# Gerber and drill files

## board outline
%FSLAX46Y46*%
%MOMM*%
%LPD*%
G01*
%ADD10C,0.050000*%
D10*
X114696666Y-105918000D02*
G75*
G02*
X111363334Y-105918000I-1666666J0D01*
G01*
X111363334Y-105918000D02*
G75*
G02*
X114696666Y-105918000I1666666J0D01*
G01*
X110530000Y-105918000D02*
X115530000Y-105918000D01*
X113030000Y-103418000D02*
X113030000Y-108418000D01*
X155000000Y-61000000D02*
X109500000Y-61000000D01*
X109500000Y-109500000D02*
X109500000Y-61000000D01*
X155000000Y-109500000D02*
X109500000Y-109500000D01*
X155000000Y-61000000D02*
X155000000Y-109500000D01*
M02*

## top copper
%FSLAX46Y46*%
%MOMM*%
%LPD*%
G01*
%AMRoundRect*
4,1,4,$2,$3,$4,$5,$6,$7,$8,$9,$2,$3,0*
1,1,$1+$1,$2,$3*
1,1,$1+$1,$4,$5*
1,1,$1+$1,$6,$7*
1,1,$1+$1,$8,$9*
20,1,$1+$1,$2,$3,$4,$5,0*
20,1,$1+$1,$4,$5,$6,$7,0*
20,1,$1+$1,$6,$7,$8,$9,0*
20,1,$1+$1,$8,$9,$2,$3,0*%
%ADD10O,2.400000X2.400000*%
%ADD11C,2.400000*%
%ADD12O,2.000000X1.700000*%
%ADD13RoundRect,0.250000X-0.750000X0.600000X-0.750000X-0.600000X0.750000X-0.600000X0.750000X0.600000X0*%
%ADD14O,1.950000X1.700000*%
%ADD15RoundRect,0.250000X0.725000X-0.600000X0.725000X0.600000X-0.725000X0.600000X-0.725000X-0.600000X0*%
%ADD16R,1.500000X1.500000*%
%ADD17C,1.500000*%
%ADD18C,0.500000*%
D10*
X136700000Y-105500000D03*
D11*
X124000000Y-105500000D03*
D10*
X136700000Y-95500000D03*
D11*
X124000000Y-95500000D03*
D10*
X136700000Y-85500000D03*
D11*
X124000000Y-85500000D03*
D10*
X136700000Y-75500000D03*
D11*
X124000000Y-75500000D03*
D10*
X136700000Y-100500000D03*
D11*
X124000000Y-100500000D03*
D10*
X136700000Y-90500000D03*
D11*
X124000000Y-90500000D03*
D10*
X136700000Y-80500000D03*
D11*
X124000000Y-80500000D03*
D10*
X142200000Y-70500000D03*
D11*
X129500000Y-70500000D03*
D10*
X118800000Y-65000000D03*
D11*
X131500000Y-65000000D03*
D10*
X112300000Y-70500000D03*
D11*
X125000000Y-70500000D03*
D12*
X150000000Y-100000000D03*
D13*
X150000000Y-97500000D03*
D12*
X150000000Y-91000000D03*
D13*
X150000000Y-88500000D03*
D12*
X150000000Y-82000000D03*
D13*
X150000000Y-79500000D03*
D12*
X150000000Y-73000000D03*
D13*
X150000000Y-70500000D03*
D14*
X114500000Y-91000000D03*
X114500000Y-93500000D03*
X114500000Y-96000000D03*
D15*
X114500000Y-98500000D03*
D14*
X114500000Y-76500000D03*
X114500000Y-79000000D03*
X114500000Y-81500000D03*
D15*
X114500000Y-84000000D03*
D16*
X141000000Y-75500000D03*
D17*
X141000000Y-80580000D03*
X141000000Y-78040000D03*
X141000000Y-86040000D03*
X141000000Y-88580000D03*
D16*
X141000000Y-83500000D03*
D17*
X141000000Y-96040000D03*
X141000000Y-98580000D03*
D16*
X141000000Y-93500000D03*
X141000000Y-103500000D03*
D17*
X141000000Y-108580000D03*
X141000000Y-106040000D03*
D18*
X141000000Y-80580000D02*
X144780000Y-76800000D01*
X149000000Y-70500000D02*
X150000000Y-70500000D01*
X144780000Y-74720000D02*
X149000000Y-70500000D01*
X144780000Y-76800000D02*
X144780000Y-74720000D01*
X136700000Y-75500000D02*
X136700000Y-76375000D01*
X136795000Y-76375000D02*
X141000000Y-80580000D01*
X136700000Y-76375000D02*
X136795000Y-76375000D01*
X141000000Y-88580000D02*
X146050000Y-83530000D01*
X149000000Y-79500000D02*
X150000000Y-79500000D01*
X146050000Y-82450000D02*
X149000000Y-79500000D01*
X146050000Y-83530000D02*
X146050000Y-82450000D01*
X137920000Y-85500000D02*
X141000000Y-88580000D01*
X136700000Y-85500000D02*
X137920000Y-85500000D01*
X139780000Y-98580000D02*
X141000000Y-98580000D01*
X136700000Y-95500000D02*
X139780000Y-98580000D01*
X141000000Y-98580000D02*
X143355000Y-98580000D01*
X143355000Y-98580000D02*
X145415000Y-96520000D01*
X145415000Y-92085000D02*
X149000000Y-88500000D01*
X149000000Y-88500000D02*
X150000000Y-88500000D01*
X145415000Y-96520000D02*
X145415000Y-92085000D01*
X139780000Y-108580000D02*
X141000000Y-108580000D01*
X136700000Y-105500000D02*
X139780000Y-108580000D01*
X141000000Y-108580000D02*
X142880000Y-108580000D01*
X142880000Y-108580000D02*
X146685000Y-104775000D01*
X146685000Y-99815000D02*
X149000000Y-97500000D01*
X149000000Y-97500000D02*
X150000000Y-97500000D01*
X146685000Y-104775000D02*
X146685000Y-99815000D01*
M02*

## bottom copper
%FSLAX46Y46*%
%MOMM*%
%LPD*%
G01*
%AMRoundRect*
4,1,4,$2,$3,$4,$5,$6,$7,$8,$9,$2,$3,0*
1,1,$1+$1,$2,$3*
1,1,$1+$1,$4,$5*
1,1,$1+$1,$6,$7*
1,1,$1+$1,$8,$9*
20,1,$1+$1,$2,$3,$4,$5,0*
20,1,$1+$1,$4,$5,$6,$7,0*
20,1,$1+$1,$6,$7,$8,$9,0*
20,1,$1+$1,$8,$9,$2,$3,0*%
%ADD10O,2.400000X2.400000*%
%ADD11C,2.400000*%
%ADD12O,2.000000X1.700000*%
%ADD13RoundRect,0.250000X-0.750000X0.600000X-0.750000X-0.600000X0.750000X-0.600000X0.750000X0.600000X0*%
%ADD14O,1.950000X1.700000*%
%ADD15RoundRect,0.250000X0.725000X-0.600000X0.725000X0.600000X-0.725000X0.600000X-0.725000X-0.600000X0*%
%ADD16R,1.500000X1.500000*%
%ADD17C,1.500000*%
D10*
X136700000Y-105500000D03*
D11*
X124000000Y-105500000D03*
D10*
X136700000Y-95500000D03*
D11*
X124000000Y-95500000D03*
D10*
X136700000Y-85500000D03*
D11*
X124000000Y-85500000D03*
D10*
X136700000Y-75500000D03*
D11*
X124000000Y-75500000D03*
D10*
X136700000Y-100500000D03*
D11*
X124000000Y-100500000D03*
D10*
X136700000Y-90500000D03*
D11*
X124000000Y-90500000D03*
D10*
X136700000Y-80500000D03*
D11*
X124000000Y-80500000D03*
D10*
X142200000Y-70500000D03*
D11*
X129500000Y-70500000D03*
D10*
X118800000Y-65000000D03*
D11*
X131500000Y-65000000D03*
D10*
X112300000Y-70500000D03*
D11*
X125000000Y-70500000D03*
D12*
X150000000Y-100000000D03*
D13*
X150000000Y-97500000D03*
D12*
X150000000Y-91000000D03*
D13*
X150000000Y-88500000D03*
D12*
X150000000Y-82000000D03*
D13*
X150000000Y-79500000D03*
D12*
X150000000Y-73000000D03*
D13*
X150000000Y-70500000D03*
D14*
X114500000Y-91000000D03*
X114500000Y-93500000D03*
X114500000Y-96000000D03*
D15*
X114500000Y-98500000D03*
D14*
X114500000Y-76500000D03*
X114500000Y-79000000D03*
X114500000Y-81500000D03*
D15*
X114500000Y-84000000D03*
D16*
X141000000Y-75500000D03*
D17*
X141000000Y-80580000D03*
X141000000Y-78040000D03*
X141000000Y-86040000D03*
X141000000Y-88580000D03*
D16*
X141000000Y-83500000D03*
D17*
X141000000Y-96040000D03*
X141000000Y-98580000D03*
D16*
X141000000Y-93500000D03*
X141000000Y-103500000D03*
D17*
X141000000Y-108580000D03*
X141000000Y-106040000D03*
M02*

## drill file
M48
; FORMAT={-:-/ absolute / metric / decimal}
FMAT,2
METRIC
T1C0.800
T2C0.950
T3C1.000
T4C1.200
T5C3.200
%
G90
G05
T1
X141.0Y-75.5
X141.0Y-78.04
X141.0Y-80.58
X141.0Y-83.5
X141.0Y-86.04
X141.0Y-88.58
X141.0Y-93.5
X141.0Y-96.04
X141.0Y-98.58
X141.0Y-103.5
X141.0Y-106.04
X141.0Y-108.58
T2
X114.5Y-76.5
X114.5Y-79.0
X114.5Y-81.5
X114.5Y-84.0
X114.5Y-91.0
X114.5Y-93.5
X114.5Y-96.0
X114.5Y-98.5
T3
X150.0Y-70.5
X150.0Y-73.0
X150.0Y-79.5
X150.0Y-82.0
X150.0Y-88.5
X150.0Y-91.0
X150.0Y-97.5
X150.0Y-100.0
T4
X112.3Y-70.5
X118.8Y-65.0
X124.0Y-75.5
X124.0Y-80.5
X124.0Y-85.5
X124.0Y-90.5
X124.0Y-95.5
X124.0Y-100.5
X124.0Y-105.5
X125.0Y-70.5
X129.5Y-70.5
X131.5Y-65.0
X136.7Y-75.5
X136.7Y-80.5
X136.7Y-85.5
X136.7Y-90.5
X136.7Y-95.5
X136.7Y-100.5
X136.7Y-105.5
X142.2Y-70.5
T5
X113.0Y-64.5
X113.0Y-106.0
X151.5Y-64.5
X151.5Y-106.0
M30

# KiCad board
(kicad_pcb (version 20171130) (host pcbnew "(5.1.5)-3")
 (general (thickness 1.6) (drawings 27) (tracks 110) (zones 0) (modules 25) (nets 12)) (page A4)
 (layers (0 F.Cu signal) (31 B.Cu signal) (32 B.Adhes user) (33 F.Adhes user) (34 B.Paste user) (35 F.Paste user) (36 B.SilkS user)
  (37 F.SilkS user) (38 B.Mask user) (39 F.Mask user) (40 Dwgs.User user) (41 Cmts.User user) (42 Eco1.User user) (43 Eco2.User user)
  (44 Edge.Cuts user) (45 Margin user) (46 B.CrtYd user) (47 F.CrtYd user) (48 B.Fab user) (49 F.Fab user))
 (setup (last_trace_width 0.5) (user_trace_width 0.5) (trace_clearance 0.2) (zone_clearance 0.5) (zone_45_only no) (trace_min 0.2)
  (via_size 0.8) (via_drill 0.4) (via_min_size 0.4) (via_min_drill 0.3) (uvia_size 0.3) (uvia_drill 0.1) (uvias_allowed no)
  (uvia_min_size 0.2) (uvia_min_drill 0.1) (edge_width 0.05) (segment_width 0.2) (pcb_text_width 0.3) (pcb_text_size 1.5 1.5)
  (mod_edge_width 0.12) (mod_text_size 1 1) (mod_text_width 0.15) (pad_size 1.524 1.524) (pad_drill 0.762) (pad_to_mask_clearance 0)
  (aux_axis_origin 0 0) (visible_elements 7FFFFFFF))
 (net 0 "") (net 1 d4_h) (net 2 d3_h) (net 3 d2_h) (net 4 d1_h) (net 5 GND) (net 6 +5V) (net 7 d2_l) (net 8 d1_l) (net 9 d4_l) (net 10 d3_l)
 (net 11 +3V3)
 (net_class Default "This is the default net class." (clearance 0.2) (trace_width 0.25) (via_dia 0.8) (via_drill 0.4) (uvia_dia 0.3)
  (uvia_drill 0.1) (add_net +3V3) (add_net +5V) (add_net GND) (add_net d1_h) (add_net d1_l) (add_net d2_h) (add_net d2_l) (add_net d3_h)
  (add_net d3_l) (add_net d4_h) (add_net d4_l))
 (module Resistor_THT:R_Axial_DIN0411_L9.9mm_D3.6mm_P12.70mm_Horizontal (layer F.Cu) (at 124 105.5)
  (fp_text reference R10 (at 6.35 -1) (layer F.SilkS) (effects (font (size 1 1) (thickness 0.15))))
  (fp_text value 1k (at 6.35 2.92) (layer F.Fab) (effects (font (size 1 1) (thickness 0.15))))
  (pad 2 thru_hole oval (at 12.7 0) (size 2.4 2.4) (drill 1.2) (layers *.Cu *.Mask) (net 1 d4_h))
  (pad 1 thru_hole circle (at 0 0) (size 2.4 2.4) (drill 1.2) (layers *.Cu *.Mask)))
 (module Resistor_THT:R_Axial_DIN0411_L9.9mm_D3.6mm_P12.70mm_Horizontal (layer F.Cu) (at 124 95.5)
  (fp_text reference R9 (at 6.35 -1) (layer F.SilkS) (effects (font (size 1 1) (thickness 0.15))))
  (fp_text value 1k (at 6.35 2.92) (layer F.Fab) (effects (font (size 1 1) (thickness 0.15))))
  (pad 2 thru_hole oval (at 12.7 0) (size 2.4 2.4) (drill 1.2) (layers *.Cu *.Mask) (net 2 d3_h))
  (pad 1 thru_hole circle (at 0 0) (size 2.4 2.4) (drill 1.2) (layers *.Cu *.Mask)))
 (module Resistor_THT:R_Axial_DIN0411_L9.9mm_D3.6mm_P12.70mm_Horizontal (layer F.Cu) (at 124 85.5)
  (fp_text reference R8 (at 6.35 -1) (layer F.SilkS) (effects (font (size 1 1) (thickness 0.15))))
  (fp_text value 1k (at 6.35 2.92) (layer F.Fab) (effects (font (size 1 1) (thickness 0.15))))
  (pad 2 thru_hole oval (at 12.7 0) (size 2.4 2.4) (drill 1.2) (layers *.Cu *.Mask) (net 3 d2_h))
  (pad 1 thru_hole circle (at 0 0) (size 2.4 2.4) (drill 1.2) (layers *.Cu *.Mask)))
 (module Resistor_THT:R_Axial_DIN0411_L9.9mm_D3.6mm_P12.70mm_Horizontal (layer F.Cu) (at 124 75.5)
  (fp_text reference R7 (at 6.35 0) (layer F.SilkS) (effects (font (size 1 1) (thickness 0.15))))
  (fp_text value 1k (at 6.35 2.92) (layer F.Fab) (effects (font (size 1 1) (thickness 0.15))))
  (pad 2 thru_hole oval (at 12.7 0) (size 2.4 2.4) (drill 1.2) (layers *.Cu *.Mask) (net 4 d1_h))
  (pad 1 thru_hole circle (at 0 0) (size 2.4 2.4) (drill 1.2) (layers *.Cu *.Mask)))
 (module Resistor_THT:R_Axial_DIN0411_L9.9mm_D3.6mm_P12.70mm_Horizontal (layer F.Cu) (at 124 100.5)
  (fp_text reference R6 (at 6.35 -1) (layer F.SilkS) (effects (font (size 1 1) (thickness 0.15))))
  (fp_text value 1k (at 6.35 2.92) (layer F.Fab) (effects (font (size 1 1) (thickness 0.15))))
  (pad 2 thru_hole oval (at 12.7 0) (size 2.4 2.4) (drill 1.2) (layers *.Cu *.Mask))
  (pad 1 thru_hole circle (at 0 0) (size 2.4 2.4) (drill 1.2) (layers *.Cu *.Mask)))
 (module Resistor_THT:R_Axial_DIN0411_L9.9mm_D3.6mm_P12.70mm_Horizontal (layer F.Cu) (at 124 90.5)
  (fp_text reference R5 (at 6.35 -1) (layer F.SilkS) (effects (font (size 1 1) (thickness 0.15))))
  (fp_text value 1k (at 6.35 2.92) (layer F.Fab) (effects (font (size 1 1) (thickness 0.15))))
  (pad 2 thru_hole oval (at 12.7 0) (size 2.4 2.4) (drill 1.2) (layers *.Cu *.Mask))
  (pad 1 thru_hole circle (at 0 0) (size 2.4 2.4) (drill 1.2) (layers *.Cu *.Mask)))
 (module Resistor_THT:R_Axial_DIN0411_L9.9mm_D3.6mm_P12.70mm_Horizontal (layer F.Cu) (at 124 80.5)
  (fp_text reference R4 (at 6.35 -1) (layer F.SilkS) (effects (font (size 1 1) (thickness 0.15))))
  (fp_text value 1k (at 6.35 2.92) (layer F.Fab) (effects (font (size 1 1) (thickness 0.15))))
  (pad 2 thru_hole oval (at 12.7 0) (size 2.4 2.4) (drill 1.2) (layers *.Cu *.Mask))
  (pad 1 thru_hole circle (at 0 0) (size 2.4 2.4) (drill 1.2) (layers *.Cu *.Mask)))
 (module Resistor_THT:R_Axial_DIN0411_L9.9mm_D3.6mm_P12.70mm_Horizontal (layer F.Cu) (at 129.5 70.5)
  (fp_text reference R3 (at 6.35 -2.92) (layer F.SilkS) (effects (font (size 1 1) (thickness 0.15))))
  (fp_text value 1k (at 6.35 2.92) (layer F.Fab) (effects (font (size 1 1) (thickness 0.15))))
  (pad 2 thru_hole oval (at 12.7 0) (size 2.4 2.4) (drill 1.2) (layers *.Cu *.Mask))
  (pad 1 thru_hole circle (at 0 0) (size 2.4 2.4) (drill 1.2) (layers *.Cu *.Mask)))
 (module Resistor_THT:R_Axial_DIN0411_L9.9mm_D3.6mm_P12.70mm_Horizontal (layer F.Cu) (at 131.5 65 180)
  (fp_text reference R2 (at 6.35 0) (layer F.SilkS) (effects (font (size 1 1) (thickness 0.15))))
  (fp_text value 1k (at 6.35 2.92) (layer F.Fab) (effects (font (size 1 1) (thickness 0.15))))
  (pad 2 thru_hole oval (at 12.7 0 180) (size 2.4 2.4) (drill 1.2) (layers *.Cu *.Mask))
  (pad 1 thru_hole circle (at 0 0 180) (size 2.4 2.4) (drill 1.2) (layers *.Cu *.Mask)))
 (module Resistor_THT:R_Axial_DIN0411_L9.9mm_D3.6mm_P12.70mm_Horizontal (layer F.Cu) (at 125 70.5 180)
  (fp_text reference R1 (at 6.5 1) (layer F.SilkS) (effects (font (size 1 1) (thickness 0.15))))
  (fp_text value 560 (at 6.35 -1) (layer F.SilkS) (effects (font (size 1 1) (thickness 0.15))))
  (pad 2 thru_hole oval (at 12.7 0 180) (size 2.4 2.4) (drill 1.2) (layers *.Cu *.Mask))
  (pad 1 thru_hole circle (at 0 0 180) (size 2.4 2.4) (drill 1.2) (layers *.Cu *.Mask)))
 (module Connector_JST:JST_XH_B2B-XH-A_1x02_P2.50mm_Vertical (layer F.Cu) (at 150 97.5 270)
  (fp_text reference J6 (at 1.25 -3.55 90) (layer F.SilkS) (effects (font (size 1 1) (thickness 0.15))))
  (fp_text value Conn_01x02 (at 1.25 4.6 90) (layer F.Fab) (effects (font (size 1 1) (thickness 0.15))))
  (pad 2 thru_hole oval (at 2.5 0 270) (size 1.7 2) (drill 1) (layers *.Cu *.Mask))
  (pad 1 thru_hole roundrect (at 0 0 270) (size 1.7 2) (drill 1) (layers *.Cu *.Mask) (roundrect_rratio 0.1470588235294118) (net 1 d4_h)))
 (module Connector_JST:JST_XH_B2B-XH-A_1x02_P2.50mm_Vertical (layer F.Cu) (at 150 88.5 270)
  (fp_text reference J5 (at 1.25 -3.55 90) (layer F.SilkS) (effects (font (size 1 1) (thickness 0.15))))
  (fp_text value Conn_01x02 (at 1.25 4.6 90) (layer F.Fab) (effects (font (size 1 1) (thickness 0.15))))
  (pad 2 thru_hole oval (at 2.5 0 270) (size 1.7 2) (drill 1) (layers *.Cu *.Mask))
  (pad 1 thru_hole roundrect (at 0 0 270) (size 1.7 2) (drill 1) (layers *.Cu *.Mask) (roundrect_rratio 0.1470588235294118) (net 2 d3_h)))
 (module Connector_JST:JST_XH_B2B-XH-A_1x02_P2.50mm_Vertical (layer F.Cu) (at 150 79.5 270)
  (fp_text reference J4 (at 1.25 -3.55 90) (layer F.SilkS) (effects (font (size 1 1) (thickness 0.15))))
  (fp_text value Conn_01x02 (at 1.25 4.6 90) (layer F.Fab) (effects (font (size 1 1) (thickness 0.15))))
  (pad 2 thru_hole oval (at 2.5 0 270) (size 1.7 2) (drill 1) (layers *.Cu *.Mask))
  (pad 1 thru_hole roundrect (at 0 0 270) (size 1.7 2) (drill 1) (layers *.Cu *.Mask) (roundrect_rratio 0.1470588235294118) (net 3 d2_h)))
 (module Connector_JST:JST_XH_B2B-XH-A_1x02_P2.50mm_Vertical (layer F.Cu) (at 150 70.5 270)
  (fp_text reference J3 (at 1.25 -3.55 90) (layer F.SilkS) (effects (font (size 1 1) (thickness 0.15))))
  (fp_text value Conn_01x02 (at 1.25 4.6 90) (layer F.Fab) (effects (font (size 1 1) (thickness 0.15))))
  (pad 2 thru_hole oval (at 2.5 0 270) (size 1.7 2) (drill 1) (layers *.Cu *.Mask))
  (pad 1 thru_hole roundrect (at 0 0 270) (size 1.7 2) (drill 1) (layers *.Cu *.Mask) (roundrect_rratio 0.1470588235294118) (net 4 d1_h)))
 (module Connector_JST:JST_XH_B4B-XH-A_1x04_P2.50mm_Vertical (layer F.Cu) (at 114.5 98.5 90)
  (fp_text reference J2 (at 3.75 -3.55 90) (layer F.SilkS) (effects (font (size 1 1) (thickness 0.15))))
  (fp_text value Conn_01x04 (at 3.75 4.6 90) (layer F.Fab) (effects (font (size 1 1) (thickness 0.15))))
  (pad 4 thru_hole oval (at 7.5 0 90) (size 1.7 1.95) (drill 0.95) (layers *.Cu *.Mask))
  (pad 3 thru_hole oval (at 5 0 90) (size 1.7 1.95) (drill 0.95) (layers *.Cu *.Mask))
  (pad 2 thru_hole oval (at 2.5 0 90) (size 1.7 1.95) (drill 0.95) (layers *.Cu *.Mask))
  (pad 1 thru_hole roundrect (at 0 0 90) (size 1.7 1.95) (drill 0.95) (layers *.Cu *.Mask) (roundrect_rratio 0.1470588235294118)))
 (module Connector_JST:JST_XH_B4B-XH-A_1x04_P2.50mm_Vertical (layer F.Cu) (at 114.5 84 90)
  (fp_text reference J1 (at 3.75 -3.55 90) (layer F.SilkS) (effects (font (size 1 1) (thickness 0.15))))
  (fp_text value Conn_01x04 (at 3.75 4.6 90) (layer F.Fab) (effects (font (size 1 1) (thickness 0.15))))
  (pad 4 thru_hole oval (at 7.5 0 90) (size 1.7 1.95) (drill 0.95) (layers *.Cu *.Mask))
  (pad 3 thru_hole oval (at 5 0 90) (size 1.7 1.95) (drill 0.95) (layers *.Cu *.Mask))
  (pad 2 thru_hole oval (at 2.5 0 90) (size 1.7 1.95) (drill 0.95) (layers *.Cu *.Mask))
  (pad 1 thru_hole roundrect (at 0 0 90) (size 1.7 1.95) (drill 0.95) (layers *.Cu *.Mask) (roundrect_rratio 0.1470588235294118)))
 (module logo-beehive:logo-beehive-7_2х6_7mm (layer F.Cu) (at 140 65)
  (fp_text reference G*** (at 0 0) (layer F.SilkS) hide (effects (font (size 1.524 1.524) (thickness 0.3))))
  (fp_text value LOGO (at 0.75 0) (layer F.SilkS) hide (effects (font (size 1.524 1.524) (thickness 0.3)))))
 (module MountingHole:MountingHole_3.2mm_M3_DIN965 (layer F.Cu) (at 113 106)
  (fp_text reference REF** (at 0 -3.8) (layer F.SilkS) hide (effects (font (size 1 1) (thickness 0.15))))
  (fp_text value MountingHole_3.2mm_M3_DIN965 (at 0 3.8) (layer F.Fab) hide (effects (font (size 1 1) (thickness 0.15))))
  (pad 1 np_thru_hole circle (at 0 0) (size 3.2 3.2) (drill 3.2) (layers *.Cu *.Mask)))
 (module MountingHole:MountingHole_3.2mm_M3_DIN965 (layer F.Cu) (at 151.5 64.5)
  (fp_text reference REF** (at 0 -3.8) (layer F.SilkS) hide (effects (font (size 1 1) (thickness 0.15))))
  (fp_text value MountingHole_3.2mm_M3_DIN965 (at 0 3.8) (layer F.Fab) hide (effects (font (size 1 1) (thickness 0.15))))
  (pad 1 np_thru_hole circle (at 0 0) (size 3.2 3.2) (drill 3.2) (layers *.Cu *.Mask)))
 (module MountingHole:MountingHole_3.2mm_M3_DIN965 (layer F.Cu) (at 113 64.5)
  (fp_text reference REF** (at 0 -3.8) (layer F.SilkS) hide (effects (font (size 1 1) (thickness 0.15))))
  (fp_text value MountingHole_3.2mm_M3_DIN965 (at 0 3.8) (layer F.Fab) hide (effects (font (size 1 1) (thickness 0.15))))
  (pad 1 np_thru_hole circle (at 0 0) (size 3.2 3.2) (drill 3.2) (layers *.Cu *.Mask)))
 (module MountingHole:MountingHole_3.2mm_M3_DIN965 (layer F.Cu) (at 151.5 106)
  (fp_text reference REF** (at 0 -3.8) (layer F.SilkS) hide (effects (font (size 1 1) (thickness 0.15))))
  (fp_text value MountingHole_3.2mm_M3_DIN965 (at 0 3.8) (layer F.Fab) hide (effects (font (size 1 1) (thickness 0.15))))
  (pad 1 np_thru_hole circle (at 0 0) (size 3.2 3.2) (drill 3.2) (layers *.Cu *.Mask)))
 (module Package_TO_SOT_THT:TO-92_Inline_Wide (layer F.Cu) (at 141 75.5 270)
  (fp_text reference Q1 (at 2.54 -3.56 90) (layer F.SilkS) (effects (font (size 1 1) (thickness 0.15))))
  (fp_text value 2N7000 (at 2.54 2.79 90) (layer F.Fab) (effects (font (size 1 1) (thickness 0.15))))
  (pad 1 thru_hole rect (at 0 0) (size 1.5 1.5) (drill 0.8) (layers *.Cu *.Mask))
  (pad 3 thru_hole circle (at 5.08 0) (size 1.5 1.5) (drill 0.8) (layers *.Cu *.Mask) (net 4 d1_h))
  (pad 2 thru_hole circle (at 2.54 0) (size 1.5 1.5) (drill 0.8) (layers *.Cu *.Mask)))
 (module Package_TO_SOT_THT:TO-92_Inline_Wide (layer F.Cu) (at 141 83.5 270)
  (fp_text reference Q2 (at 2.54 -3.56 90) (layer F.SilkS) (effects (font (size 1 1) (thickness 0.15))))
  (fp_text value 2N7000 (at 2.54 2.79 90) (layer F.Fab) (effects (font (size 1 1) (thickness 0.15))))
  (pad 2 thru_hole circle (at 2.54 0) (size 1.5 1.5) (drill 0.8) (layers *.Cu *.Mask))
  (pad 3 thru_hole circle (at 5.08 0) (size 1.5 1.5) (drill 0.8) (layers *.Cu *.Mask) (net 3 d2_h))
  (pad 1 thru_hole rect (at 0 0) (size 1.5 1.5) (drill 0.8) (layers *.Cu *.Mask)))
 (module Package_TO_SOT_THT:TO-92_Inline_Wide (layer F.Cu) (at 141 93.5 270)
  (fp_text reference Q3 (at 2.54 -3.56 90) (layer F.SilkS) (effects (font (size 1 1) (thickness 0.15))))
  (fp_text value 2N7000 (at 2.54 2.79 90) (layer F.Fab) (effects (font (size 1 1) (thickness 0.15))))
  (pad 2 thru_hole circle (at 2.54 0) (size 1.5 1.5) (drill 0.8) (layers *.Cu *.Mask))
  (pad 3 thru_hole circle (at 5.08 0) (size 1.5 1.5) (drill 0.8) (layers *.Cu *.Mask) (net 2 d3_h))
  (pad 1 thru_hole rect (at 0 0) (size 1.5 1.5) (drill 0.8) (layers *.Cu *.Mask)))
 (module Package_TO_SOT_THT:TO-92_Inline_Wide (layer F.Cu) (at 141 103.5 270)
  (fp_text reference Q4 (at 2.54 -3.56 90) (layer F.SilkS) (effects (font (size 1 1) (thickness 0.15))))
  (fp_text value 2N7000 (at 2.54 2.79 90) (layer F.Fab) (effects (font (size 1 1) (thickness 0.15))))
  (pad 1 thru_hole rect (at 0 0) (size 1.5 1.5) (drill 0.8) (layers *.Cu *.Mask))
  (pad 3 thru_hole circle (at 5.08 0) (size 1.5 1.5) (drill 0.8) (layers *.Cu *.Mask) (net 1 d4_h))
  (pad 2 thru_hole circle (at 2.54 0) (size 1.5 1.5) (drill 0.8) (layers *.Cu *.Mask)))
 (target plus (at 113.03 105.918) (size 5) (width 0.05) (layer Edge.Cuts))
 (gr_line (start 155 61) (end 109.5 61) (layer Edge.Cuts) (width 0.05))
 (gr_line (start 109.5 109.5) (end 109.5 61) (layer Edge.Cuts) (width 0.05))
 (gr_line (start 155 109.5) (end 109.5 109.5) (layer Edge.Cuts) (width 0.05))
 (gr_line (start 155 61) (end 155 109.5) (layer Edge.Cuts) (width 0.05))
 (segment (start 141 80.58) (end 144.78 76.8) (width 0.5) (layer F.Cu) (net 4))
 (segment (start 149 70.5) (end 150 70.5) (width 0.5) (layer F.Cu) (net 4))
 (segment (start 144.78 74.72) (end 149 70.5) (width 0.5) (layer F.Cu) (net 4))
 (segment (start 144.78 76.8) (end 144.78 74.72) (width 0.5) (layer F.Cu) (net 4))
 (segment (start 136.7 75.5) (end 136.7 76.375) (width 0.5) (layer F.Cu) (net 4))
 (segment (start 136.795 76.375) (end 141 80.58) (width 0.5) (layer F.Cu) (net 4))
 (segment (start 136.7 76.375) (end 136.795 76.375) (width 0.5) (layer F.Cu) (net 4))
 (segment (start 141 88.58) (end 146.05 83.53) (width 0.5) (layer F.Cu) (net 3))
 (segment (start 149 79.5) (end 150 79.5) (width 0.5) (layer F.Cu) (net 3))
 (segment (start 146.05 82.45) (end 149 79.5) (width 0.5) (layer F.Cu) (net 3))
 (segment (start 146.05 83.53) (end 146.05 82.45) (width 0.5) (layer F.Cu) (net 3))
 (segment (start 137.92 85.5) (end 141 88.58) (width 0.5) (layer F.Cu) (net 3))
 (segment (start 136.7 85.5) (end 137.92 85.5) (width 0.5) (layer F.Cu) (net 3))
 (segment (start 139.78 98.58) (end 141 98.58) (width 0.5) (layer F.Cu) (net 2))
 (segment (start 136.7 95.5) (end 139.78 98.58) (width 0.5) (layer F.Cu) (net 2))
 (segment (start 141 98.58) (end 143.355 98.58) (width 0.5) (layer F.Cu) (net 2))
 (segment (start 143.355 98.58) (end 145.415 96.52) (width 0.5) (layer F.Cu) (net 2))
 (segment (start 145.415 92.085) (end 149 88.5) (width 0.5) (layer F.Cu) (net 2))
 (segment (start 149 88.5) (end 150 88.5) (width 0.5) (layer F.Cu) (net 2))
 (segment (start 145.415 96.52) (end 145.415 92.085) (width 0.5) (layer F.Cu) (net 2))
 (segment (start 139.78 108.58) (end 141 108.58) (width 0.5) (layer F.Cu) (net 1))
 (segment (start 136.7 105.5) (end 139.78 108.58) (width 0.5) (layer F.Cu) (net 1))
 (segment (start 141 108.58) (end 142.88 108.58) (width 0.5) (layer F.Cu) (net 1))
 (segment (start 142.88 108.58) (end 146.685 104.775) (width 0.5) (layer F.Cu) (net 1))
 (segment (start 146.685 99.815) (end 149 97.5) (width 0.5) (layer F.Cu) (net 1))
 (segment (start 149 97.5) (end 150 97.5) (width 0.5) (layer F.Cu) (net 1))
 (segment (start 146.685 104.775) (end 146.685 99.815) (width 0.5) (layer F.Cu) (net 1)))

